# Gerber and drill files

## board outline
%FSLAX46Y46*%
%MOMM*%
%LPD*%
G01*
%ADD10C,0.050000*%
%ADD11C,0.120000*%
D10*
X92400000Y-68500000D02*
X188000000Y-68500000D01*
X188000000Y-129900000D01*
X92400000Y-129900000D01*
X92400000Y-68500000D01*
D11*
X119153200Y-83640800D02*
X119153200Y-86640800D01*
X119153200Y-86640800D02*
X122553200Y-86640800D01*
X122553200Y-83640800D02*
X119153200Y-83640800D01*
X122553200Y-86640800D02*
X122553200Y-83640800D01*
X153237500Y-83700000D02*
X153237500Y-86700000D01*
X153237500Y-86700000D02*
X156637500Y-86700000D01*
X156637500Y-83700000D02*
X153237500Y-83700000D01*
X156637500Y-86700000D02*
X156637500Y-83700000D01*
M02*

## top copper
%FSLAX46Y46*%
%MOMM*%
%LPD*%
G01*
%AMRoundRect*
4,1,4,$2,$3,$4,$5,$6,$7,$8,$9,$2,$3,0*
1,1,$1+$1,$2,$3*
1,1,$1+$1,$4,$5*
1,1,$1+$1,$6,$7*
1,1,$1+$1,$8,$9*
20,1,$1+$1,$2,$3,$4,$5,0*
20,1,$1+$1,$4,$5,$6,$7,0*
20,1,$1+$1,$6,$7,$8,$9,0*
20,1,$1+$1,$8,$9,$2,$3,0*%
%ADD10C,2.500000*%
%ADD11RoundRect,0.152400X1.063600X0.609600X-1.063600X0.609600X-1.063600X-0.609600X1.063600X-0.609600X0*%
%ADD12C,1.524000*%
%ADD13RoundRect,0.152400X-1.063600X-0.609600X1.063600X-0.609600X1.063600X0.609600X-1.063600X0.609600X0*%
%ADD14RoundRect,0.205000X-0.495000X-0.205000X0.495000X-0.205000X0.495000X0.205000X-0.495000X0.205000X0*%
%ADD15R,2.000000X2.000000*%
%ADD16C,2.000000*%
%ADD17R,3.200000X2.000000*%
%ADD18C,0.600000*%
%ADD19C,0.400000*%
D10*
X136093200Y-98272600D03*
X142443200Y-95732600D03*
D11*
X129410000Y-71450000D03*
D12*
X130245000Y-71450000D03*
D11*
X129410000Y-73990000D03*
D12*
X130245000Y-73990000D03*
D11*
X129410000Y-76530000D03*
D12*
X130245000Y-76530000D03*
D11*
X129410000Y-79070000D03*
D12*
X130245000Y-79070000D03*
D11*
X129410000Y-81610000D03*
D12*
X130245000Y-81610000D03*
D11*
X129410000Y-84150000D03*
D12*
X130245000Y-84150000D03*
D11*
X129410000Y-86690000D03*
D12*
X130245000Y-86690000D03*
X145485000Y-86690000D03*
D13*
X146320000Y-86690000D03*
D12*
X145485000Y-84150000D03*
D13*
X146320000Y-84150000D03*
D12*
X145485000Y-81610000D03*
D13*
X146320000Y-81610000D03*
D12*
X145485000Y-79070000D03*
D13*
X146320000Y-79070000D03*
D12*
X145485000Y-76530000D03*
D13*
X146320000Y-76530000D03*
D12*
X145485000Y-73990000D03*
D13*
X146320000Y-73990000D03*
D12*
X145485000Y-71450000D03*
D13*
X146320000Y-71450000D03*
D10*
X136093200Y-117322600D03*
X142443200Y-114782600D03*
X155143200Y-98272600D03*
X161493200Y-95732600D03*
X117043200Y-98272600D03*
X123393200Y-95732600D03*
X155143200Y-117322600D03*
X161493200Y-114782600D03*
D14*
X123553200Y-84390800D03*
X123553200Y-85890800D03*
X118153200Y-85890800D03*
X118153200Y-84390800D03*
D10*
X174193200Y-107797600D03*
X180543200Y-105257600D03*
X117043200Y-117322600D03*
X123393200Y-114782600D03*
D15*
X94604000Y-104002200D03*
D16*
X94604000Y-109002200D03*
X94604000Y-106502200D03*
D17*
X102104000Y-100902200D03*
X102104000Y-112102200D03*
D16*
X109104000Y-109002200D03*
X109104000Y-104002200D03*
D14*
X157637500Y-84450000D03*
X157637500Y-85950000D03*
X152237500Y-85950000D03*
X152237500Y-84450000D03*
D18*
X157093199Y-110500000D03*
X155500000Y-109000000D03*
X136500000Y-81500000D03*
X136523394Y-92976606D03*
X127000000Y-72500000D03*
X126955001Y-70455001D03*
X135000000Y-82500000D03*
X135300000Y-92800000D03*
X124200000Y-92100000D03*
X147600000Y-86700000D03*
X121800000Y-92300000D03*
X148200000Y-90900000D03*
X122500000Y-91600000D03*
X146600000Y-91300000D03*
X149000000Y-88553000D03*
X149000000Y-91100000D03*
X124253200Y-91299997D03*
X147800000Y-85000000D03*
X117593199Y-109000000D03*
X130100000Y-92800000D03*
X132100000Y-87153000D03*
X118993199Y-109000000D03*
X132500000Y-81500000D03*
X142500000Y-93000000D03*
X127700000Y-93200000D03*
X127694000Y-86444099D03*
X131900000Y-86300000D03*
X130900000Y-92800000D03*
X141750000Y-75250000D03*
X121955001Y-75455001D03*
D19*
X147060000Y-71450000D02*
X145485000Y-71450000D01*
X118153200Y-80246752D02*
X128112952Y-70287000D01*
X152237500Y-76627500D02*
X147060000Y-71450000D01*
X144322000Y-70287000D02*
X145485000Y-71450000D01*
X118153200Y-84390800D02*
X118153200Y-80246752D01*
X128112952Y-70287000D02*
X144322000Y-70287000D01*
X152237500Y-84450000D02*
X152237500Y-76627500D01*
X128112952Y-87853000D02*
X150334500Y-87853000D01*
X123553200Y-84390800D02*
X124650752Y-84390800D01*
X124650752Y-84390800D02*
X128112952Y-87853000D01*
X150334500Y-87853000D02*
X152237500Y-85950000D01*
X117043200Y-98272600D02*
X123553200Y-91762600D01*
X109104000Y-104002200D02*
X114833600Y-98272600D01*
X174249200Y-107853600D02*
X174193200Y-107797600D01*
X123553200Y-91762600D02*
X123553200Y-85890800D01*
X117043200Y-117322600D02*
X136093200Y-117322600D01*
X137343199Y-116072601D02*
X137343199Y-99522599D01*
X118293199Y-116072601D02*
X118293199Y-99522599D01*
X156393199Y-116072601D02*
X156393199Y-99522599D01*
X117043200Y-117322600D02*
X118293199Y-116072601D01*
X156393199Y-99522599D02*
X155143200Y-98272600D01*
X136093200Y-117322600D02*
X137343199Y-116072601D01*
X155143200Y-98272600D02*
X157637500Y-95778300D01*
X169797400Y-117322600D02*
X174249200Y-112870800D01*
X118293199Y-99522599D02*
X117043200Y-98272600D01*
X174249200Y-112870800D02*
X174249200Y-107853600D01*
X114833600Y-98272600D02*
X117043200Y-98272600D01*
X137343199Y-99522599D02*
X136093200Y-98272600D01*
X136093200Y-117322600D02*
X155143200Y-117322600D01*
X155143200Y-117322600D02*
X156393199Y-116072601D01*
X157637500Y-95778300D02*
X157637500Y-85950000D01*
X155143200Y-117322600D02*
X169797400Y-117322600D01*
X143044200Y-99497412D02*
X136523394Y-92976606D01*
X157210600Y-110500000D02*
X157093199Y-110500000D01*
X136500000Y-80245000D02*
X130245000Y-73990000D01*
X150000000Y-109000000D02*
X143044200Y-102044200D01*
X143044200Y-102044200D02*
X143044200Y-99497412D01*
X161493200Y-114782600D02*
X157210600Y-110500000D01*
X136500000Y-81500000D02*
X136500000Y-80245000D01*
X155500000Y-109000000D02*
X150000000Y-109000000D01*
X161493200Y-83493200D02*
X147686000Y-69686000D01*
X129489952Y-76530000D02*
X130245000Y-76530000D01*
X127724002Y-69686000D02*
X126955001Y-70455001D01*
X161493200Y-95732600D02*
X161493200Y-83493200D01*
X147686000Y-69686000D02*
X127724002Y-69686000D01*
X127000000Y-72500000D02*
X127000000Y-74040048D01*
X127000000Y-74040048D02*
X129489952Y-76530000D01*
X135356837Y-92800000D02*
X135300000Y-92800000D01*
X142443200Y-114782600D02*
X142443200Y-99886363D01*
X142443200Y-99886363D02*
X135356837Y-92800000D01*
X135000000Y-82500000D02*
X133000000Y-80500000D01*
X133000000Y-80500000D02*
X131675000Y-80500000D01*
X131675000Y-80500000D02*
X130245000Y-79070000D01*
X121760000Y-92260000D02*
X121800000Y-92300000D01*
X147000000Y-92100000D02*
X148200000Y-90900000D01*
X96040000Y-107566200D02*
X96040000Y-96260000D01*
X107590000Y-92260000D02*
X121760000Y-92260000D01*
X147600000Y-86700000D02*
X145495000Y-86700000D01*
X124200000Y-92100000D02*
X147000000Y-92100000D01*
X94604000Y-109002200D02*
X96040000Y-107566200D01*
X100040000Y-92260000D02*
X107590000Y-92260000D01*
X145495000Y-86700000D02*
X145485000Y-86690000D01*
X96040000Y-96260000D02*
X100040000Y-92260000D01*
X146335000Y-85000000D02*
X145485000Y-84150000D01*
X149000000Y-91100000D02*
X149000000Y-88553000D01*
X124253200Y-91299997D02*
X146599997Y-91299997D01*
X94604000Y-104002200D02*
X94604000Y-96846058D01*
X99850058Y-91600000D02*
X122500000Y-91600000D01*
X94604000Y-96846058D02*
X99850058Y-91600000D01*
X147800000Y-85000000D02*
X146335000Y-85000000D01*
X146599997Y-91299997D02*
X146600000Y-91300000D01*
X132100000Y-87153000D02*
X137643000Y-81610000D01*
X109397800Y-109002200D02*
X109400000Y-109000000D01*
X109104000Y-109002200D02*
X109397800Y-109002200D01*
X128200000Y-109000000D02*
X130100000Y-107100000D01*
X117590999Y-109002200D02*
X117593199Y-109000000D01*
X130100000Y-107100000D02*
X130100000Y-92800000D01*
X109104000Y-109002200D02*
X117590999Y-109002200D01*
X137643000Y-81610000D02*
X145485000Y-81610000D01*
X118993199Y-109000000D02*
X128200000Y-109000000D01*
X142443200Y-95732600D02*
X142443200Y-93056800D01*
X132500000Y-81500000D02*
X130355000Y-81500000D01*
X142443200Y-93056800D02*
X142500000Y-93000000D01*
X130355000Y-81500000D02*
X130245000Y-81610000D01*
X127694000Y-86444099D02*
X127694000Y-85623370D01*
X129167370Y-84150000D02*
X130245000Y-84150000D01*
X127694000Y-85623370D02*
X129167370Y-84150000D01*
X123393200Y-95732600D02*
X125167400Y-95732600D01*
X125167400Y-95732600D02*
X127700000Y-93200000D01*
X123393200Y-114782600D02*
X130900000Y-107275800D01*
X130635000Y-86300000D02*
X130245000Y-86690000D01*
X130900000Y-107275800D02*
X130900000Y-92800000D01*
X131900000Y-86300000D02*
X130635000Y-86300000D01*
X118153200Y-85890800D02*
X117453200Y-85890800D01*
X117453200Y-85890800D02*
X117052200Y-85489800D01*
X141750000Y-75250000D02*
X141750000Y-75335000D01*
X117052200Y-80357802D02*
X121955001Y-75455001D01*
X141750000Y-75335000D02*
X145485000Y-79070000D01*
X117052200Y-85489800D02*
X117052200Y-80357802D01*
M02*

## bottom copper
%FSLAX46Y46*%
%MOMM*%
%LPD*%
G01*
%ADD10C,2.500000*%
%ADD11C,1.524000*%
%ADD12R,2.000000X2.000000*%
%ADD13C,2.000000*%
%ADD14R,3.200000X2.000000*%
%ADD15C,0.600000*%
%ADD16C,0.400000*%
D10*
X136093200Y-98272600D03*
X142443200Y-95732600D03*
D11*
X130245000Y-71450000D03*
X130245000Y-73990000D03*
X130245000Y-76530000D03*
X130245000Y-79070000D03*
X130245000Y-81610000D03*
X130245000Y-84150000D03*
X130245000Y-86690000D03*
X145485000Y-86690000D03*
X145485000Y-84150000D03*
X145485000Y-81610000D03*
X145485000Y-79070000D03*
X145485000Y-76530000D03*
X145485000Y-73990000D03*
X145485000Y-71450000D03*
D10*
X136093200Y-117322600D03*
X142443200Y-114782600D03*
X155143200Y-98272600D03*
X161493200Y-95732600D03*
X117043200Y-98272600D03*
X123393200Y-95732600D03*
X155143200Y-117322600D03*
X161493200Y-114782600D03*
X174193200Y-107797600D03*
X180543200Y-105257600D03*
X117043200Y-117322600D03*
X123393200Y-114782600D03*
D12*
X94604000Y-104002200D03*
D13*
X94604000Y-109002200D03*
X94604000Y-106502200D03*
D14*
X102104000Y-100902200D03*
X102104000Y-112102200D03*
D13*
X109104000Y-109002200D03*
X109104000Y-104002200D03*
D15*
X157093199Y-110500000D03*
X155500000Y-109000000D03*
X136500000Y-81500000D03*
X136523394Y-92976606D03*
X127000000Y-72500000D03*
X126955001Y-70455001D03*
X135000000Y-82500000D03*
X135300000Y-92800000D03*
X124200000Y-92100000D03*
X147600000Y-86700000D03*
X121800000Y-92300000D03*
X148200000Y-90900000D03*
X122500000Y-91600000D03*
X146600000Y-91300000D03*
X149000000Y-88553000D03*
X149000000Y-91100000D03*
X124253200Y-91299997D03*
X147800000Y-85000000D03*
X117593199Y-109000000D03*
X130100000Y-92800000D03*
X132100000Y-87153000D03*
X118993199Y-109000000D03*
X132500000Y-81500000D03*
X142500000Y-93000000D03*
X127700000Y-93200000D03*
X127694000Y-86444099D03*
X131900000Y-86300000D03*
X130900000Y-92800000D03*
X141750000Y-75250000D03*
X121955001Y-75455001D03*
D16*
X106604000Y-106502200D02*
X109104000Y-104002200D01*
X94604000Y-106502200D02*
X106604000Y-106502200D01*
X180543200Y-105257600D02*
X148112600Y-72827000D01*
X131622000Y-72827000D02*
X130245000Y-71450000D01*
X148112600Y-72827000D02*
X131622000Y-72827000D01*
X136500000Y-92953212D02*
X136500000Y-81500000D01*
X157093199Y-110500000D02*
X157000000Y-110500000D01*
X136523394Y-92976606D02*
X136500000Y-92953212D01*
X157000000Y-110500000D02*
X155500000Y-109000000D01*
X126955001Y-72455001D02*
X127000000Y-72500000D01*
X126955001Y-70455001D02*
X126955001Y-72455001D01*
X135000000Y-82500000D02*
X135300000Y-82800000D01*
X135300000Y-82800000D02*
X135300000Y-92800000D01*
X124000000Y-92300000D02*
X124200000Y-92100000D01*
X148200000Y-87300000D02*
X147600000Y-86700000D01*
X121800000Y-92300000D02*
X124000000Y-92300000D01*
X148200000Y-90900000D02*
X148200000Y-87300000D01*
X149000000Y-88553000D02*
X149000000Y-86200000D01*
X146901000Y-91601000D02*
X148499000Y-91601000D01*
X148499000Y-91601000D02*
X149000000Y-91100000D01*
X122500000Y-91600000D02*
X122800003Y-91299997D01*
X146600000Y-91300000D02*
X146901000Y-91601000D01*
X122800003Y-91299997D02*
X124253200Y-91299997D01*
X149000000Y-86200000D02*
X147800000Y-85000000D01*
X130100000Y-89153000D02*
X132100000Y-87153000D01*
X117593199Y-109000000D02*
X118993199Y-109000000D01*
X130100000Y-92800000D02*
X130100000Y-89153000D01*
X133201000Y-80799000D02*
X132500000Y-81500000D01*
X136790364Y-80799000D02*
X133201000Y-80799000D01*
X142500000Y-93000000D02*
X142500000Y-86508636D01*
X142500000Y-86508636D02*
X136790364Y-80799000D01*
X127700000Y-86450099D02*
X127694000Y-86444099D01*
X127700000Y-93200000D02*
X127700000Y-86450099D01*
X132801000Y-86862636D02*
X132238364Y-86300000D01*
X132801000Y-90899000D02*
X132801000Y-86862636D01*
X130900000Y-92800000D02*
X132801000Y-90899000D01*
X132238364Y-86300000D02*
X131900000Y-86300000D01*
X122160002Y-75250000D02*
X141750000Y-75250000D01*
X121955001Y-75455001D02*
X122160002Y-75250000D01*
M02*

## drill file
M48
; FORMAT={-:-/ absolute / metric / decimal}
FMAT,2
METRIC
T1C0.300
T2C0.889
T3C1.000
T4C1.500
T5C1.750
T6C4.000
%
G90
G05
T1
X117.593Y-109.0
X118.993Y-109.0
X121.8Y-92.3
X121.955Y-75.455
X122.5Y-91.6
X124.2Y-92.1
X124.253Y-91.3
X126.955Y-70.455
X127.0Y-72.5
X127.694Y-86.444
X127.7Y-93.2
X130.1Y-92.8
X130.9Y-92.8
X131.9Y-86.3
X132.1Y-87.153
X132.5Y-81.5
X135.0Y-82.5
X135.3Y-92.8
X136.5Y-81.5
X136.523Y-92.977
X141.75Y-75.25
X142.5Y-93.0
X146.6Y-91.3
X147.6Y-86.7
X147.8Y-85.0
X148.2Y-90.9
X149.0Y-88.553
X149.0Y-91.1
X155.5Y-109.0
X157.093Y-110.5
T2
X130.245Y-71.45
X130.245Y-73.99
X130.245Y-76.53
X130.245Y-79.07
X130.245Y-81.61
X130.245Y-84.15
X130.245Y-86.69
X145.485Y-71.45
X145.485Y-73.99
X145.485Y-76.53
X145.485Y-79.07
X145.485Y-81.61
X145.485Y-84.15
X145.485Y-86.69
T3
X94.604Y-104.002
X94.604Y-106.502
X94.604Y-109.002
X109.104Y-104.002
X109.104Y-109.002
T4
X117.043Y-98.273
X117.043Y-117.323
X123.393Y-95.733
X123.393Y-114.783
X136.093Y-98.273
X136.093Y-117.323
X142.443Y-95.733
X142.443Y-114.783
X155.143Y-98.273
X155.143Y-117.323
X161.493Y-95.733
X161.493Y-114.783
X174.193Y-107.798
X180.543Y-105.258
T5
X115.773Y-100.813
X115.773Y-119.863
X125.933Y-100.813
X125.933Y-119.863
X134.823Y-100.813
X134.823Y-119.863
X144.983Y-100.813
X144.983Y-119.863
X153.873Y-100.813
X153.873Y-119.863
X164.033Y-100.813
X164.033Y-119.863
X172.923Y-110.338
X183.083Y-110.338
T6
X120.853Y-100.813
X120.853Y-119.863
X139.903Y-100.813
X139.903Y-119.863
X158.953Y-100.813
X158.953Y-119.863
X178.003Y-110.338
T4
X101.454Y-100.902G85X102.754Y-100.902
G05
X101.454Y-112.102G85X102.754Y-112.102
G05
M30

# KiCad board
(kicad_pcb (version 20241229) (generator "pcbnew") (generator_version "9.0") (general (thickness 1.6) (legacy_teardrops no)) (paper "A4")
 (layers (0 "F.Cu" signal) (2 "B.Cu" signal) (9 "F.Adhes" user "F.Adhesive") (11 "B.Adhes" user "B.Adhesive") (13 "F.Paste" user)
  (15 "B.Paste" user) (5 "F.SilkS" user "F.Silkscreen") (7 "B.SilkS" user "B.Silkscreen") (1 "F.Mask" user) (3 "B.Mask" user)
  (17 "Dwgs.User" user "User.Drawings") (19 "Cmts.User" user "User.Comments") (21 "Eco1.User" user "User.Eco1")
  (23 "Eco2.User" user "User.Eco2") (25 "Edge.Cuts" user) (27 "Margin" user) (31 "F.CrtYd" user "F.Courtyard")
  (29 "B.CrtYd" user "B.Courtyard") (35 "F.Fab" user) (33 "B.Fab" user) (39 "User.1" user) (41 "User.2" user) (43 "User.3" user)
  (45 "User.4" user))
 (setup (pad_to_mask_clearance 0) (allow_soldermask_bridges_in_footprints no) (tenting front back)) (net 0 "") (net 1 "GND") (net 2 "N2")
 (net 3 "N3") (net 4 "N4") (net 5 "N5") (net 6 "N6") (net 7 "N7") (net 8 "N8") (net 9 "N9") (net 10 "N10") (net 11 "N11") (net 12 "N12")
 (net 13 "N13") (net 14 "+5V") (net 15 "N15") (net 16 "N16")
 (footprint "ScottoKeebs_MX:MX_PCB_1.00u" (layer "F.Cu") (at 139.9032 100.8126)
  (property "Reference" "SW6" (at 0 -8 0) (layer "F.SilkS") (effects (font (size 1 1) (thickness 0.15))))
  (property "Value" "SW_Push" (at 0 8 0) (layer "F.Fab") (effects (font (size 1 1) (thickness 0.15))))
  (pad "" np_thru_hole circle (at -5.08 0) (size 1.75 1.75) (drill 1.75) (layers "*.Cu" "*.Mask"))
  (pad "" np_thru_hole circle (at 0 0) (size 4 4) (drill 4) (layers "*.Cu" "*.Mask"))
  (pad "" np_thru_hole circle (at 5.08 0) (size 1.75 1.75) (drill 1.75) (layers "*.Cu" "*.Mask"))
  (pad "1" thru_hole circle (at -3.81 -2.54) (size 2.5 2.5) (drill 1.5) (layers "*.Cu" "*.Mask") (remove_unused_layers no) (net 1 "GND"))
  (pad "2" thru_hole circle (at 2.54 -5.08) (size 2.5 2.5) (drill 1.5) (layers "*.Cu" "*.Mask") (remove_unused_layers no) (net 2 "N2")))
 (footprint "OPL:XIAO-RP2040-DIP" (layer "F.Cu") (at 137.865 79.07)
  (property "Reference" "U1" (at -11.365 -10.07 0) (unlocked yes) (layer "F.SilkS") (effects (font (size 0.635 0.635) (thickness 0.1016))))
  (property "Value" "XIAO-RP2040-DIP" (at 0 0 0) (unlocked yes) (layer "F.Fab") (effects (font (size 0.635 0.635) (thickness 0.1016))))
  (pad "1" smd roundrect (at -8.455 -7.62 180) (size 2.432 1.524) (layers "F.Cu" "F.Mask") (roundrect_rratio 0.1) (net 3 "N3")
   (thermal_bridge_angle 45))
  (pad "1" thru_hole circle (at -7.62 -7.62 180) (size 1.524 1.524) (drill 0.889) (layers "*.Cu" "*.Mask") (remove_unused_layers no)
   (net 3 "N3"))
  (pad "2" smd roundrect (at -8.455 -5.08 180) (size 2.432 1.524) (layers "F.Cu" "F.Mask") (roundrect_rratio 0.1) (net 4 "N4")
   (thermal_bridge_angle 45))
  (pad "2" thru_hole circle (at -7.62 -5.08 180) (size 1.524 1.524) (drill 0.889) (layers "*.Cu" "*.Mask") (remove_unused_layers no)
   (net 4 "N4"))
  (pad "3" smd roundrect (at -8.455 -2.54 180) (size 2.432 1.524) (layers "F.Cu" "F.Mask") (roundrect_rratio 0.1) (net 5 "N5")
   (thermal_bridge_angle 45))
  (pad "3" thru_hole circle (at -7.62 -2.54 180) (size 1.524 1.524) (drill 0.889) (layers "*.Cu" "*.Mask") (remove_unused_layers no)
   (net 5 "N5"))
  (pad "4" smd roundrect (at -8.455 0 180) (size 2.432 1.524) (layers "F.Cu" "F.Mask") (roundrect_rratio 0.1) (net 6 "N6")
   (thermal_bridge_angle 45))
  (pad "4" thru_hole circle (at -7.62 0 180) (size 1.524 1.524) (drill 0.889) (layers "*.Cu" "*.Mask") (remove_unused_layers no)
   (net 6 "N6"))
  (pad "5" smd roundrect (at -8.455 2.54 180) (size 2.432 1.524) (layers "F.Cu" "F.Mask") (roundrect_rratio 0.1) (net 2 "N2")
   (thermal_bridge_angle 45))
  (pad "5" thru_hole circle (at -7.62 2.54 180) (size 1.524 1.524) (drill 0.889) (layers "*.Cu" "*.Mask") (remove_unused_layers no)
   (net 2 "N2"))
  (pad "6" smd roundrect (at -8.455 5.08 180) (size 2.432 1.524) (layers "F.Cu" "F.Mask") (roundrect_rratio 0.1) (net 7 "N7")
   (thermal_bridge_angle 45))
  (pad "6" thru_hole circle (at -7.62 5.08 180) (size 1.524 1.524) (drill 0.889) (layers "*.Cu" "*.Mask") (remove_unused_layers no)
   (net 7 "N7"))
  (pad "7" smd roundrect (at -8.455 7.62 180) (size 2.432 1.524) (layers "F.Cu" "F.Mask") (roundrect_rratio 0.1) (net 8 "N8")
   (thermal_bridge_angle 45))
  (pad "7" thru_hole circle (at -7.62 7.62 180) (size 1.524 1.524) (drill 0.889) (layers "*.Cu" "*.Mask") (remove_unused_layers no)
   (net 8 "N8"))
  (pad "8" thru_hole circle (at 7.62 7.62) (size 1.524 1.524) (drill 0.889) (layers "*.Cu" "*.Mask") (remove_unused_layers no) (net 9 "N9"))
  (pad "8" smd roundrect (at 8.455 7.62) (size 2.432 1.524) (layers "F.Cu" "F.Mask") (roundrect_rratio 0.1) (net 9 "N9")
   (thermal_bridge_angle 45))
  (pad "9" thru_hole circle (at 7.62 5.08) (size 1.524 1.524) (drill 0.889) (layers "*.Cu" "*.Mask") (remove_unused_layers no)
   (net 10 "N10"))
  (pad "9" smd roundrect (at 8.455 5.08) (size 2.432 1.524) (layers "F.Cu" "F.Mask") (roundrect_rratio 0.1) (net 10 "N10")
   (thermal_bridge_angle 45))
  (pad "10" thru_hole circle (at 7.62 2.54) (size 1.524 1.524) (drill 0.889) (layers "*.Cu" "*.Mask") (remove_unused_layers no)
   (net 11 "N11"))
  (pad "10" smd roundrect (at 8.455 2.54) (size 2.432 1.524) (layers "F.Cu" "F.Mask") (roundrect_rratio 0.1) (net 11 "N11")
   (thermal_bridge_angle 45))
  (pad "11" thru_hole circle (at 7.62 0) (size 1.524 1.524) (drill 0.889) (layers "*.Cu" "*.Mask") (remove_unused_layers no) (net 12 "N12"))
  (pad "11" smd roundrect (at 8.455 0) (size 2.432 1.524) (layers "F.Cu" "F.Mask") (roundrect_rratio 0.1) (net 12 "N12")
   (thermal_bridge_angle 45))
  (pad "12" thru_hole circle (at 7.62 -2.54) (size 1.524 1.524) (drill 0.889) (layers "*.Cu" "*.Mask") (remove_unused_layers no)
   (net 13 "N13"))
  (pad "12" smd roundrect (at 8.455 -2.54) (size 2.432 1.524) (layers "F.Cu" "F.Mask") (roundrect_rratio 0.1) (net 13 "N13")
   (thermal_bridge_angle 45))
  (pad "13" thru_hole circle (at 7.62 -5.08) (size 1.524 1.524) (drill 0.889) (layers "*.Cu" "*.Mask") (remove_unused_layers no)
   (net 1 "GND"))
  (pad "13" smd roundrect (at 8.455 -5.08) (size 2.432 1.524) (layers "F.Cu" "F.Mask") (roundrect_rratio 0.1) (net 1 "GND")
   (thermal_bridge_angle 45))
  (pad "14" thru_hole circle (at 7.62 -7.62) (size 1.524 1.524) (drill 0.889) (layers "*.Cu" "*.Mask") (remove_unused_layers no)
   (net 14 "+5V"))
  (pad "14" smd roundrect (at 8.455 -7.62) (size 2.432 1.524) (layers "F.Cu" "F.Mask") (roundrect_rratio 0.1) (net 14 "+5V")
   (thermal_bridge_angle 45)))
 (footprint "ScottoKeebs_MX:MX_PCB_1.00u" (layer "F.Cu") (at 139.9032 119.8626)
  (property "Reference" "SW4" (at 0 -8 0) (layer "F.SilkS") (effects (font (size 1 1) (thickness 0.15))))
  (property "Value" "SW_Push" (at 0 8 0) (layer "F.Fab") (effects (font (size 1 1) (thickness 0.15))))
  (pad "" np_thru_hole circle (at -5.08 0) (size 1.75 1.75) (drill 1.75) (layers "*.Cu" "*.Mask"))
  (pad "" np_thru_hole circle (at 0 0) (size 4 4) (drill 4) (layers "*.Cu" "*.Mask"))
  (pad "" np_thru_hole circle (at 5.08 0) (size 1.75 1.75) (drill 1.75) (layers "*.Cu" "*.Mask"))
  (pad "1" thru_hole circle (at -3.81 -2.54) (size 2.5 2.5) (drill 1.5) (layers "*.Cu" "*.Mask") (remove_unused_layers no) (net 1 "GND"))
  (pad "2" thru_hole circle (at 2.54 -5.08) (size 2.5 2.5) (drill 1.5) (layers "*.Cu" "*.Mask") (remove_unused_layers no) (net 6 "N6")))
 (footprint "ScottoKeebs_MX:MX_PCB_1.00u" (layer "F.Cu") (at 158.9532 100.8126)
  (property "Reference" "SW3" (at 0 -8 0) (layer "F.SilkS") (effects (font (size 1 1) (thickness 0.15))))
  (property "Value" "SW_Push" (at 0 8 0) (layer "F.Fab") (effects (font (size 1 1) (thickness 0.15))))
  (pad "" np_thru_hole circle (at -5.08 0) (size 1.75 1.75) (drill 1.75) (layers "*.Cu" "*.Mask"))
  (pad "" np_thru_hole circle (at 0 0) (size 4 4) (drill 4) (layers "*.Cu" "*.Mask"))
  (pad "" np_thru_hole circle (at 5.08 0) (size 1.75 1.75) (drill 1.75) (layers "*.Cu" "*.Mask"))
  (pad "1" thru_hole circle (at -3.81 -2.54) (size 2.5 2.5) (drill 1.5) (layers "*.Cu" "*.Mask") (remove_unused_layers no) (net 1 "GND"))
  (pad "2" thru_hole circle (at 2.54 -5.08) (size 2.5 2.5) (drill 1.5) (layers "*.Cu" "*.Mask") (remove_unused_layers no) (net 5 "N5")))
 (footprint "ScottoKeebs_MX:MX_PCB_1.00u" (layer "F.Cu") (at 120.8532 100.8126)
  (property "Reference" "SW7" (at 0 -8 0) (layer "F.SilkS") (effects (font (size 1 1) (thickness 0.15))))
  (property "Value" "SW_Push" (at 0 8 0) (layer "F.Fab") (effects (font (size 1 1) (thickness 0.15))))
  (pad "" np_thru_hole circle (at -5.08 0) (size 1.75 1.75) (drill 1.75) (layers "*.Cu" "*.Mask"))
  (pad "" np_thru_hole circle (at 0 0) (size 4 4) (drill 4) (layers "*.Cu" "*.Mask"))
  (pad "" np_thru_hole circle (at 5.08 0) (size 1.75 1.75) (drill 1.75) (layers "*.Cu" "*.Mask"))
  (pad "1" thru_hole circle (at -3.81 -2.54) (size 2.5 2.5) (drill 1.5) (layers "*.Cu" "*.Mask") (remove_unused_layers no) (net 1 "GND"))
  (pad "2" thru_hole circle (at 2.54 -5.08) (size 2.5 2.5) (drill 1.5) (layers "*.Cu" "*.Mask") (remove_unused_layers no) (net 7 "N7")))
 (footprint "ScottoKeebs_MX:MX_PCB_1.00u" (layer "F.Cu") (at 158.9532 119.8626)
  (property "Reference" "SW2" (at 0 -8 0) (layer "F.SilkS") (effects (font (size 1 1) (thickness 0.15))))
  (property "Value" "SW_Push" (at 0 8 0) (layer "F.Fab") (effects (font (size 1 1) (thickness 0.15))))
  (pad "" np_thru_hole circle (at -5.08 0) (size 1.75 1.75) (drill 1.75) (layers "*.Cu" "*.Mask"))
  (pad "" np_thru_hole circle (at 0 0) (size 4 4) (drill 4) (layers "*.Cu" "*.Mask"))
  (pad "" np_thru_hole circle (at 5.08 0) (size 1.75 1.75) (drill 1.75) (layers "*.Cu" "*.Mask"))
  (pad "1" thru_hole circle (at -3.81 -2.54) (size 2.5 2.5) (drill 1.5) (layers "*.Cu" "*.Mask") (remove_unused_layers no) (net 1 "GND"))
  (pad "2" thru_hole circle (at 2.54 -5.08) (size 2.5 2.5) (drill 1.5) (layers "*.Cu" "*.Mask") (remove_unused_layers no) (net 4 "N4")))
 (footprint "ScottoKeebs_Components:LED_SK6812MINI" (layer "F.Cu") (at 120.8532 85.1408)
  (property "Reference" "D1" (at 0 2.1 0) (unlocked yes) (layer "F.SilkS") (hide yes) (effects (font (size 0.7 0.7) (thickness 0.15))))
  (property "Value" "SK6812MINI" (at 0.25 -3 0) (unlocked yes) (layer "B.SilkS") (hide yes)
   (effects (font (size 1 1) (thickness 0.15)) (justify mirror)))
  (fp_line (start -1.7 -1.5) (end -1.7 1.5) (stroke (width 0.12) (type solid)) (layer "Edge.Cuts"))
  (fp_line (start -1.7 1.5) (end 1.7 1.5) (stroke (width 0.12) (type solid)) (layer "Edge.Cuts"))
  (fp_line (start 1.7 -1.5) (end -1.7 -1.5) (stroke (width 0.12) (type solid)) (layer "Edge.Cuts"))
  (fp_line (start 1.7 1.5) (end 1.7 -1.5) (stroke (width 0.12) (type solid)) (layer "Edge.Cuts"))
  (pad "1" smd roundrect (at 2.7 -0.75) (size 1.4 0.82) (layers "F.Cu" "F.Mask" "F.Paste") (roundrect_rratio 0.25) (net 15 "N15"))
  (pad "2" smd roundrect (at 2.7 0.75) (size 1.4 0.82) (layers "F.Cu" "F.Mask" "F.Paste") (roundrect_rratio 0.25) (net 1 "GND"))
  (pad "3" smd roundrect (at -2.7 0.75) (size 1.4 0.82) (layers "F.Cu" "F.Mask" "F.Paste") (roundrect_rratio 0.25) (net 12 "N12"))
  (pad "4" smd roundrect (at -2.7 -0.75) (size 1.4 0.82) (layers "F.Cu" "F.Mask" "F.Paste") (roundrect_rratio 0.25) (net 14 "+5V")))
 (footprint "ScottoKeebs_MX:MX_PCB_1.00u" (layer "F.Cu") (at 178.0032 110.3376)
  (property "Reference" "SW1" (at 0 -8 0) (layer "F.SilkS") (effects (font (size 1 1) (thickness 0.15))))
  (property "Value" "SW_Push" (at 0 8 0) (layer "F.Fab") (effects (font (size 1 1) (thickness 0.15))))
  (pad "" np_thru_hole circle (at -5.08 0) (size 1.75 1.75) (drill 1.75) (layers "*.Cu" "*.Mask"))
  (pad "" np_thru_hole circle (at 0 0) (size 4 4) (drill 4) (layers "*.Cu" "*.Mask"))
  (pad "" np_thru_hole circle (at 5.08 0) (size 1.75 1.75) (drill 1.75) (layers "*.Cu" "*.Mask"))
  (pad "1" thru_hole circle (at -3.81 -2.54) (size 2.5 2.5) (drill 1.5) (layers "*.Cu" "*.Mask") (remove_unused_layers no) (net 1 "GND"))
  (pad "2" thru_hole circle (at 2.54 -5.08) (size 2.5 2.5) (drill 1.5) (layers "*.Cu" "*.Mask") (remove_unused_layers no) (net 3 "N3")))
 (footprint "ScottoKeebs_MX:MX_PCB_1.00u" (layer "F.Cu") (at 120.8532 119.8626)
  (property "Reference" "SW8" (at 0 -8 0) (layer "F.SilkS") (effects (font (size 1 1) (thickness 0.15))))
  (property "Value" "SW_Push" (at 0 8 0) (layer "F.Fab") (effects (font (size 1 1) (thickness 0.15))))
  (pad "" np_thru_hole circle (at -5.08 0) (size 1.75 1.75) (drill 1.75) (layers "*.Cu" "*.Mask"))
  (pad "" np_thru_hole circle (at 0 0) (size 4 4) (drill 4) (layers "*.Cu" "*.Mask"))
  (pad "" np_thru_hole circle (at 5.08 0) (size 1.75 1.75) (drill 1.75) (layers "*.Cu" "*.Mask"))
  (pad "1" thru_hole circle (at -3.81 -2.54) (size 2.5 2.5) (drill 1.5) (layers "*.Cu" "*.Mask") (remove_unused_layers no) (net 1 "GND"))
  (pad "2" thru_hole circle (at 2.54 -5.08) (size 2.5 2.5) (drill 1.5) (layers "*.Cu" "*.Mask") (remove_unused_layers no) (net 8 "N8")))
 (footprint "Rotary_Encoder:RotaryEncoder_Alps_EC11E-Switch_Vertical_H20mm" (layer "F.Cu") (at 94.604 104.0022)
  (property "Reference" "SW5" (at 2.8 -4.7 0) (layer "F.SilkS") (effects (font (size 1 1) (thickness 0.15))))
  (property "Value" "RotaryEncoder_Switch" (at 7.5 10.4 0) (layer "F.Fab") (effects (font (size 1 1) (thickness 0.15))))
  (pad "A" thru_hole rect (at 0 0) (size 2 2) (drill 1) (layers "*.Cu" "*.Mask") (remove_unused_layers no) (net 10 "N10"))
  (pad "B" thru_hole circle (at 0 5) (size 2 2) (drill 1) (layers "*.Cu" "*.Mask") (remove_unused_layers no) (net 9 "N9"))
  (pad "C" thru_hole circle (at 0 2.5) (size 2 2) (drill 1) (layers "*.Cu" "*.Mask") (remove_unused_layers no) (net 1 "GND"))
  (pad "MP" thru_hole rect (at 7.5 -3.1) (size 3.2 2) (drill oval 2.8 1.5) (layers "*.Cu" "*.Mask") (remove_unused_layers no))
  (pad "MP" thru_hole rect (at 7.5 8.1) (size 3.2 2) (drill oval 2.8 1.5) (layers "*.Cu" "*.Mask") (remove_unused_layers no))
  (pad "S1" thru_hole circle (at 14.5 5) (size 2 2) (drill 1) (layers "*.Cu" "*.Mask") (remove_unused_layers no) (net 11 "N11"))
  (pad "S2" thru_hole circle (at 14.5 0) (size 2 2) (drill 1) (layers "*.Cu" "*.Mask") (remove_unused_layers no) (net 1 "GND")))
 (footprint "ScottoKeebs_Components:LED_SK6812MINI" (layer "F.Cu") (at 154.9375 85.2)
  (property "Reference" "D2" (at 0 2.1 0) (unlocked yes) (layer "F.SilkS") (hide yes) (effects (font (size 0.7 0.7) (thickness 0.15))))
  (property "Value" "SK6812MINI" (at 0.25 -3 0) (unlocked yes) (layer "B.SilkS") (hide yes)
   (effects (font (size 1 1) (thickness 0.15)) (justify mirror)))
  (fp_line (start -1.7 -1.5) (end -1.7 1.5) (stroke (width 0.12) (type solid)) (layer "Edge.Cuts"))
  (fp_line (start -1.7 1.5) (end 1.7 1.5) (stroke (width 0.12) (type solid)) (layer "Edge.Cuts"))
  (fp_line (start 1.7 -1.5) (end -1.7 -1.5) (stroke (width 0.12) (type solid)) (layer "Edge.Cuts"))
  (fp_line (start 1.7 1.5) (end 1.7 -1.5) (stroke (width 0.12) (type solid)) (layer "Edge.Cuts"))
  (pad "1" smd roundrect (at 2.7 -0.75) (size 1.4 0.82) (layers "F.Cu" "F.Mask" "F.Paste") (roundrect_rratio 0.25) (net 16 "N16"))
  (pad "2" smd roundrect (at 2.7 0.75) (size 1.4 0.82) (layers "F.Cu" "F.Mask" "F.Paste") (roundrect_rratio 0.25) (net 1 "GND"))
  (pad "3" smd roundrect (at -2.7 0.75) (size 1.4 0.82) (layers "F.Cu" "F.Mask" "F.Paste") (roundrect_rratio 0.25) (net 15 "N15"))
  (pad "4" smd roundrect (at -2.7 -0.75) (size 1.4 0.82) (layers "F.Cu" "F.Mask" "F.Paste") (roundrect_rratio 0.25) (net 14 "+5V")))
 (gr_rect (start 92.4 68.5) (end 188 129.9) (stroke (width 0.05) (type default)) (fill no) (layer "Edge.Cuts"))
 (segment (start 147.06 71.45) (end 145.485 71.45) (width 0.4) (layer "F.Cu") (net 14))
 (segment (start 118.1532 80.246752) (end 128.112952 70.287) (width 0.4) (layer "F.Cu") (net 14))
 (segment (start 152.2375 76.6275) (end 147.06 71.45) (width 0.4) (layer "F.Cu") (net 14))
 (segment (start 144.322 70.287) (end 145.485 71.45) (width 0.4) (layer "F.Cu") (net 14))
 (segment (start 118.1532 84.3908) (end 118.1532 80.246752) (width 0.4) (layer "F.Cu") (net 14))
 (segment (start 128.112952 70.287) (end 144.322 70.287) (width 0.4) (layer "F.Cu") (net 14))
 (segment (start 152.2375 84.45) (end 152.2375 76.6275) (width 0.4) (layer "F.Cu") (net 14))
 (segment (start 128.112952 87.853) (end 150.3345 87.853) (width 0.4) (layer "F.Cu") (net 15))
 (segment (start 123.5532 84.3908) (end 124.650752 84.3908) (width 0.4) (layer "F.Cu") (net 15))
 (segment (start 124.650752 84.3908) (end 128.112952 87.853) (width 0.4) (layer "F.Cu") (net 15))
 (segment (start 150.3345 87.853) (end 152.2375 85.95) (width 0.4) (layer "F.Cu") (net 15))
 (segment (start 117.0432 98.2726) (end 123.5532 91.7626) (width 0.4) (layer "F.Cu") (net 1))
 (segment (start 109.104 104.0022) (end 114.8336 98.2726) (width 0.4) (layer "F.Cu") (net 1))
 (segment (start 174.2492 107.8536) (end 174.1932 107.7976) (width 0.4) (layer "F.Cu") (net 1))
 (segment (start 123.5532 91.7626) (end 123.5532 85.8908) (width 0.4) (layer "F.Cu") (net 1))
 (segment (start 117.0432 117.3226) (end 136.0932 117.3226) (width 0.4) (layer "F.Cu") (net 1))
 (segment (start 137.343199 116.072601) (end 137.343199 99.522599) (width 0.4) (layer "F.Cu") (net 1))
 (segment (start 118.293199 116.072601) (end 118.293199 99.522599) (width 0.4) (layer "F.Cu") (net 1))
 (segment (start 156.393199 116.072601) (end 156.393199 99.522599) (width 0.4) (layer "F.Cu") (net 1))
 (segment (start 117.0432 117.3226) (end 118.293199 116.072601) (width 0.4) (layer "F.Cu") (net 1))
 (segment (start 156.393199 99.522599) (end 155.1432 98.2726) (width 0.4) (layer "F.Cu") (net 1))
 (segment (start 136.0932 117.3226) (end 137.343199 116.072601) (width 0.4) (layer "F.Cu") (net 1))
 (segment (start 155.1432 98.2726) (end 157.6375 95.7783) (width 0.4) (layer "F.Cu") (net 1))
 (segment (start 169.7974 117.3226) (end 174.2492 112.8708) (width 0.4) (layer "F.Cu") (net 1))
 (segment (start 118.293199 99.522599) (end 117.0432 98.2726) (width 0.4) (layer "F.Cu") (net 1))
 (segment (start 174.2492 112.8708) (end 174.2492 107.8536) (width 0.4) (layer "F.Cu") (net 1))
 (segment (start 114.8336 98.2726) (end 117.0432 98.2726) (width 0.4) (layer "F.Cu") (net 1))
 (segment (start 137.343199 99.522599) (end 136.0932 98.2726) (width 0.4) (layer "F.Cu") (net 1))
 (segment (start 136.0932 117.3226) (end 155.1432 117.3226) (width 0.4) (layer "F.Cu") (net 1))
 (segment (start 155.1432 117.3226) (end 156.393199 116.072601) (width 0.4) (layer "F.Cu") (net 1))
 (segment (start 157.6375 95.7783) (end 157.6375 85.95) (width 0.4) (layer "F.Cu") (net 1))
 (segment (start 155.1432 117.3226) (end 169.7974 117.3226) (width 0.4) (layer "F.Cu") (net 1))
 (segment (start 106.604 106.5022) (end 109.104 104.0022) (width 0.4) (layer "B.Cu") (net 1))
 (segment (start 94.604 106.5022) (end 106.604 106.5022) (width 0.4) (layer "B.Cu") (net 1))
 (segment (start 180.5432 105.2576) (end 148.1126 72.827) (width 0.4) (layer "B.Cu") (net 3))
 (segment (start 131.622 72.827) (end 130.245 71.45) (width 0.4) (layer "B.Cu") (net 3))
 (segment (start 148.1126 72.827) (end 131.622 72.827) (width 0.4) (layer "B.Cu") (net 3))
 (segment (start 143.0442 99.497412) (end 136.523394 92.976606) (width 0.4) (layer "F.Cu") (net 4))
 (segment (start 157.2106 110.5) (end 157.093199 110.5) (width 0.4) (layer "F.Cu") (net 4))
 (segment (start 136.5 80.245) (end 130.245 73.99) (width 0.4) (layer "F.Cu") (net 4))
 (segment (start 150 109) (end 143.0442 102.0442) (width 0.4) (layer "F.Cu") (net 4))
 (segment (start 143.0442 102.0442) (end 143.0442 99.497412) (width 0.4) (layer "F.Cu") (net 4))
 (segment (start 161.4932 114.7826) (end 157.2106 110.5) (width 0.4) (layer "F.Cu") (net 4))
 (segment (start 136.5 81.5) (end 136.5 80.245) (width 0.4) (layer "F.Cu") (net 4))
 (segment (start 155.5 109) (end 150 109) (width 0.4) (layer "F.Cu") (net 4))
 (via (at 157.093199 110.5) (size 0.6) (drill 0.3) (layers "F.Cu" "B.Cu") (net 4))
 (via (at 155.5 109) (size 0.6) (drill 0.3) (layers "F.Cu" "B.Cu") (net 4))
 (via (at 136.5 81.5) (size 0.6) (drill 0.3) (layers "F.Cu" "B.Cu") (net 4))
 (via (at 136.523394 92.976606) (size 0.6) (drill 0.3) (layers "F.Cu" "B.Cu") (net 4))
 (segment (start 136.5 92.953212) (end 136.5 81.5) (width 0.4) (layer "B.Cu") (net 4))
 (segment (start 157.093199 110.5) (end 157 110.5) (width 0.4) (layer "B.Cu") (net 4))
 (segment (start 136.523394 92.976606) (end 136.5 92.953212) (width 0.4) (layer "B.Cu") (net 4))
 (segment (start 157 110.5) (end 155.5 109) (width 0.4) (layer "B.Cu") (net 4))
 (segment (start 161.4932 83.4932) (end 147.686 69.686) (width 0.4) (layer "F.Cu") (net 5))
 (segment (start 129.489952 76.53) (end 130.245 76.53) (width 0.4) (layer "F.Cu") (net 5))
 (segment (start 127.724002 69.686) (end 126.955001 70.455001) (width 0.4) (layer "F.Cu") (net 5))
 (segment (start 161.4932 95.7326) (end 161.4932 83.4932) (width 0.4) (layer "F.Cu") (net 5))
 (segment (start 147.686 69.686) (end 127.724002 69.686) (width 0.4) (layer "F.Cu") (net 5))
 (segment (start 127 72.5) (end 127 74.040048) (width 0.4) (layer "F.Cu") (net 5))
 (segment (start 127 74.040048) (end 129.489952 76.53) (width 0.4) (layer "F.Cu") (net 5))
 (via (at 127 72.5) (size 0.6) (drill 0.3) (layers "F.Cu" "B.Cu") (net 5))
 (via (at 126.955001 70.455001) (size 0.6) (drill 0.3) (layers "F.Cu" "B.Cu") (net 5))
 (segment (start 126.955001 72.455001) (end 127 72.5) (width 0.4) (layer "B.Cu") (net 5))
 (segment (start 126.955001 70.455001) (end 126.955001 72.455001) (width 0.4) (layer "B.Cu") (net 5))
 (segment (start 135.356837 92.8) (end 135.3 92.8) (width 0.4) (layer "F.Cu") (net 6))
 (segment (start 142.4432 114.7826) (end 142.4432 99.886363) (width 0.4) (layer "F.Cu") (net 6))
 (segment (start 142.4432 99.886363) (end 135.356837 92.8) (width 0.4) (layer "F.Cu") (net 6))
 (segment (start 135 82.5) (end 133 80.5) (width 0.4) (layer "F.Cu") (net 6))
 (segment (start 133 80.5) (end 131.675 80.5) (width 0.4) (layer "F.Cu") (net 6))
 (segment (start 131.675 80.5) (end 130.245 79.07) (width 0.4) (layer "F.Cu") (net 6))
 (via (at 135 82.5) (size 0.6) (drill 0.3) (layers "F.Cu" "B.Cu") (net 6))
 (via (at 135.3 92.8) (size 0.6) (drill 0.3) (layers "F.Cu" "B.Cu") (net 6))
 (segment (start 135 82.5) (end 135.3 82.8) (width 0.4) (layer "B.Cu") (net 6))
 (segment (start 135.3 82.8) (end 135.3 92.8) (width 0.4) (layer "B.Cu") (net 6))
 (segment (start 121.76 92.26) (end 121.8 92.3) (width 0.4) (layer "F.Cu") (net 9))
 (segment (start 147 92.1) (end 148.2 90.9) (width 0.4) (layer "F.Cu") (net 9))
 (segment (start 96.04 107.5662) (end 96.04 96.26) (width 0.4) (layer "F.Cu") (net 9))
 (segment (start 107.59 92.26) (end 121.76 92.26) (width 0.4) (layer "F.Cu") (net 9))
 (segment (start 147.6 86.7) (end 145.495 86.7) (width 0.4) (layer "F.Cu") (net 9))
 (segment (start 124.2 92.1) (end 147 92.1) (width 0.4) (layer "F.Cu") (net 9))
 (segment (start 94.604 109.0022) (end 96.04 107.5662) (width 0.4) (layer "F.Cu") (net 9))
 (segment (start 100.04 92.26) (end 107.59 92.26) (width 0.4) (layer "F.Cu") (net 9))
 (segment (start 145.495 86.7) (end 145.485 86.69) (width 0.4) (layer "F.Cu") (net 9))
 (segment (start 96.04 96.26) (end 100.04 92.26) (width 0.4) (layer "F.Cu") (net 9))
 (via (at 124.2 92.1) (size 0.6) (drill 0.3) (layers "F.Cu" "B.Cu") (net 9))
 (via (at 147.6 86.7) (size 0.6) (drill 0.3) (layers "F.Cu" "B.Cu") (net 9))
 (via (at 121.8 92.3) (size 0.6) (drill 0.3) (layers "F.Cu" "B.Cu") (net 9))
 (via (at 148.2 90.9) (size 0.6) (drill 0.3) (layers "F.Cu" "B.Cu") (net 9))
 (segment (start 124 92.3) (end 124.2 92.1) (width 0.4) (layer "B.Cu") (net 9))
 (segment (start 148.2 87.3) (end 147.6 86.7) (width 0.4) (layer "B.Cu") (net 9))
 (segment (start 121.8 92.3) (end 124 92.3) (width 0.4) (layer "B.Cu") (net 9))
 (segment (start 148.2 90.9) (end 148.2 87.3) (width 0.4) (layer "B.Cu") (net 9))
 (segment (start 146.335 85) (end 145.485 84.15) (width 0.4) (layer "F.Cu") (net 10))
 (segment (start 149 91.1) (end 149 88.553) (width 0.4) (layer "F.Cu") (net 10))
 (segment (start 124.2532 91.299997) (end 146.599997 91.299997) (width 0.4) (layer "F.Cu") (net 10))
 (segment (start 94.604 104.0022) (end 94.604 96.846058) (width 0.4) (layer "F.Cu") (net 10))
 (segment (start 99.850058 91.6) (end 122.5 91.6) (width 0.4) (layer "F.Cu") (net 10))
 (segment (start 94.604 96.846058) (end 99.850058 91.6) (width 0.4) (layer "F.Cu") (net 10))
 (segment (start 147.8 85) (end 146.335 85) (width 0.4) (layer "F.Cu") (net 10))
 (segment (start 146.599997 91.299997) (end 146.6 91.3) (width 0.4) (layer "F.Cu") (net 10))
 (via (at 122.5 91.6) (size 0.6) (drill 0.3) (layers "F.Cu" "B.Cu") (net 10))
 (via (at 146.6 91.3) (size 0.6) (drill 0.3) (layers "F.Cu" "B.Cu") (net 10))
 (via (at 149 88.553) (size 0.6) (drill 0.3) (layers "F.Cu" "B.Cu") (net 10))
 (via (at 149 91.1) (size 0.6) (drill 0.3) (layers "F.Cu" "B.Cu") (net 10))
 (via (at 124.2532 91.299997) (size 0.6) (drill 0.3) (layers "F.Cu" "B.Cu") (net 10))
 (via (at 147.8 85) (size 0.6) (drill 0.3) (layers "F.Cu" "B.Cu") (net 10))
 (segment (start 149 88.553) (end 149 86.2) (width 0.4) (layer "B.Cu") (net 10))
 (segment (start 146.901 91.601) (end 148.499 91.601) (width 0.4) (layer "B.Cu") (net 10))
 (segment (start 148.499 91.601) (end 149 91.1) (width 0.4) (layer "B.Cu") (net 10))
 (segment (start 122.5 91.6) (end 122.800003 91.299997) (width 0.4) (layer "B.Cu") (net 10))
 (segment (start 146.6 91.3) (end 146.901 91.601) (width 0.4) (layer "B.Cu") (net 10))
 (segment (start 122.800003 91.299997) (end 124.2532 91.299997) (width 0.4) (layer "B.Cu") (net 10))
 (segment (start 149 86.2) (end 147.8 85) (width 0.4) (layer "B.Cu") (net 10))
 (segment (start 132.1 87.153) (end 137.643 81.61) (width 0.4) (layer "F.Cu") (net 11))
 (segment (start 109.3978 109.0022) (end 109.4 109) (width 0.4) (layer "F.Cu") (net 11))
 (segment (start 109.104 109.0022) (end 109.3978 109.0022) (width 0.4) (layer "F.Cu") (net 11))
 (segment (start 128.2 109) (end 130.1 107.1) (width 0.4) (layer "F.Cu") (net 11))
 (segment (start 117.590999 109.0022) (end 117.593199 109) (width 0.4) (layer "F.Cu") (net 11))
 (segment (start 130.1 107.1) (end 130.1 92.8) (width 0.4) (layer "F.Cu") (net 11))
 (segment (start 109.104 109.0022) (end 117.590999 109.0022) (width 0.4) (layer "F.Cu") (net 11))
 (segment (start 137.643 81.61) (end 145.485 81.61) (width 0.4) (layer "F.Cu") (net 11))
 (segment (start 118.993199 109) (end 128.2 109) (width 0.4) (layer "F.Cu") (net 11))
 (via (at 117.593199 109) (size 0.6) (drill 0.3) (layers "F.Cu" "B.Cu") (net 11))
 (via (at 130.1 92.8) (size 0.6) (drill 0.3) (layers "F.Cu" "B.Cu") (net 11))
 (via (at 132.1 87.153) (size 0.6) (drill 0.3) (layers "F.Cu" "B.Cu") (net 11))
 (via (at 118.993199 109) (size 0.6) (drill 0.3) (layers "F.Cu" "B.Cu") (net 11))
 (segment (start 130.1 89.153) (end 132.1 87.153) (width 0.4) (layer "B.Cu") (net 11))
 (segment (start 117.593199 109) (end 118.993199 109) (width 0.4) (layer "B.Cu") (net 11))
 (segment (start 130.1 92.8) (end 130.1 89.153) (width 0.4) (layer "B.Cu") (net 11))
 (segment (start 142.4432 95.7326) (end 142.4432 93.0568) (width 0.4) (layer "F.Cu") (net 2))
 (segment (start 132.5 81.5) (end 130.355 81.5) (width 0.4) (layer "F.Cu") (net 2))
 (segment (start 142.4432 93.0568) (end 142.5 93) (width 0.4) (layer "F.Cu") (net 2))
 (segment (start 130.355 81.5) (end 130.245 81.61) (width 0.4) (layer "F.Cu") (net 2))
 (via (at 132.5 81.5) (size 0.6) (drill 0.3) (layers "F.Cu" "B.Cu") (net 2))
 (via (at 142.5 93) (size 0.6) (drill 0.3) (layers "F.Cu" "B.Cu") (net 2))
 (segment (start 133.201 80.799) (end 132.5 81.5) (width 0.4) (layer "B.Cu") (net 2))
 (segment (start 136.790364 80.799) (end 133.201 80.799) (width 0.4) (layer "B.Cu") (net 2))
 (segment (start 142.5 93) (end 142.5 86.508636) (width 0.4) (layer "B.Cu") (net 2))
 (segment (start 142.5 86.508636) (end 136.790364 80.799) (width 0.4) (layer "B.Cu") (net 2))
 (segment (start 127.694 86.444099) (end 127.694 85.62337) (width 0.4) (layer "F.Cu") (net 7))
 (segment (start 129.16737 84.15) (end 130.245 84.15) (width 0.4) (layer "F.Cu") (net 7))
 (segment (start 127.694 85.62337) (end 129.16737 84.15) (width 0.4) (layer "F.Cu") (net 7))
 (segment (start 123.3932 95.7326) (end 125.1674 95.7326) (width 0.4) (layer "F.Cu") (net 7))
 (segment (start 125.1674 95.7326) (end 127.7 93.2) (width 0.4) (layer "F.Cu") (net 7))
 (via (at 127.7 93.2) (size 0.6) (drill 0.3) (layers "F.Cu" "B.Cu") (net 7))
 (via (at 127.694 86.444099) (size 0.6) (drill 0.3) (layers "F.Cu" "B.Cu") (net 7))
 (segment (start 127.7 86.450099) (end 127.694 86.444099) (width 0.4) (layer "B.Cu") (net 7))
 (segment (start 127.7 93.2) (end 127.7 86.450099) (width 0.4) (layer "B.Cu") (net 7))
 (segment (start 123.3932 114.7826) (end 130.9 107.2758) (width 0.4) (layer "F.Cu") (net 8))
 (segment (start 130.635 86.3) (end 130.245 86.69) (width 0.4) (layer "F.Cu") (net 8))
 (segment (start 130.9 107.2758) (end 130.9 92.8) (width 0.4) (layer "F.Cu") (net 8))
 (segment (start 131.9 86.3) (end 130.635 86.3) (width 0.4) (layer "F.Cu") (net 8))
 (via (at 131.9 86.3) (size 0.6) (drill 0.3) (layers "F.Cu" "B.Cu") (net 8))
 (via (at 130.9 92.8) (size 0.6) (drill 0.3) (layers "F.Cu" "B.Cu") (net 8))
 (segment (start 132.801 86.862636) (end 132.238364 86.3) (width 0.4) (layer "B.Cu") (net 8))
 (segment (start 132.801 90.899) (end 132.801 86.862636) (width 0.4) (layer "B.Cu") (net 8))
 (segment (start 130.9 92.8) (end 132.801 90.899) (width 0.4) (layer "B.Cu") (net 8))
 (segment (start 132.238364 86.3) (end 131.9 86.3) (width 0.4) (layer "B.Cu") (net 8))
 (segment (start 118.1532 85.8908) (end 117.4532 85.8908) (width 0.4) (layer "F.Cu") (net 12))
 (segment (start 117.4532 85.8908) (end 117.0522 85.4898) (width 0.4) (layer "F.Cu") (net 12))
 (segment (start 141.75 75.25) (end 141.75 75.335) (width 0.4) (layer "F.Cu") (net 12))
 (segment (start 117.0522 80.357802) (end 121.955001 75.455001) (width 0.4) (layer "F.Cu") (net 12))
 (segment (start 141.75 75.335) (end 145.485 79.07) (width 0.4) (layer "F.Cu") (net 12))
 (segment (start 117.0522 85.4898) (end 117.0522 80.357802) (width 0.4) (layer "F.Cu") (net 12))
 (via (at 141.75 75.25) (size 0.6) (drill 0.3) (layers "F.Cu" "B.Cu") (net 12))
 (via (at 121.955001 75.455001) (size 0.6) (drill 0.3) (layers "F.Cu" "B.Cu") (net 12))
 (segment (start 122.160002 75.25) (end 141.75 75.25) (width 0.4) (layer "B.Cu") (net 12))
 (segment (start 121.955001 75.455001) (end 122.160002 75.25) (width 0.4) (layer "B.Cu") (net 12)))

